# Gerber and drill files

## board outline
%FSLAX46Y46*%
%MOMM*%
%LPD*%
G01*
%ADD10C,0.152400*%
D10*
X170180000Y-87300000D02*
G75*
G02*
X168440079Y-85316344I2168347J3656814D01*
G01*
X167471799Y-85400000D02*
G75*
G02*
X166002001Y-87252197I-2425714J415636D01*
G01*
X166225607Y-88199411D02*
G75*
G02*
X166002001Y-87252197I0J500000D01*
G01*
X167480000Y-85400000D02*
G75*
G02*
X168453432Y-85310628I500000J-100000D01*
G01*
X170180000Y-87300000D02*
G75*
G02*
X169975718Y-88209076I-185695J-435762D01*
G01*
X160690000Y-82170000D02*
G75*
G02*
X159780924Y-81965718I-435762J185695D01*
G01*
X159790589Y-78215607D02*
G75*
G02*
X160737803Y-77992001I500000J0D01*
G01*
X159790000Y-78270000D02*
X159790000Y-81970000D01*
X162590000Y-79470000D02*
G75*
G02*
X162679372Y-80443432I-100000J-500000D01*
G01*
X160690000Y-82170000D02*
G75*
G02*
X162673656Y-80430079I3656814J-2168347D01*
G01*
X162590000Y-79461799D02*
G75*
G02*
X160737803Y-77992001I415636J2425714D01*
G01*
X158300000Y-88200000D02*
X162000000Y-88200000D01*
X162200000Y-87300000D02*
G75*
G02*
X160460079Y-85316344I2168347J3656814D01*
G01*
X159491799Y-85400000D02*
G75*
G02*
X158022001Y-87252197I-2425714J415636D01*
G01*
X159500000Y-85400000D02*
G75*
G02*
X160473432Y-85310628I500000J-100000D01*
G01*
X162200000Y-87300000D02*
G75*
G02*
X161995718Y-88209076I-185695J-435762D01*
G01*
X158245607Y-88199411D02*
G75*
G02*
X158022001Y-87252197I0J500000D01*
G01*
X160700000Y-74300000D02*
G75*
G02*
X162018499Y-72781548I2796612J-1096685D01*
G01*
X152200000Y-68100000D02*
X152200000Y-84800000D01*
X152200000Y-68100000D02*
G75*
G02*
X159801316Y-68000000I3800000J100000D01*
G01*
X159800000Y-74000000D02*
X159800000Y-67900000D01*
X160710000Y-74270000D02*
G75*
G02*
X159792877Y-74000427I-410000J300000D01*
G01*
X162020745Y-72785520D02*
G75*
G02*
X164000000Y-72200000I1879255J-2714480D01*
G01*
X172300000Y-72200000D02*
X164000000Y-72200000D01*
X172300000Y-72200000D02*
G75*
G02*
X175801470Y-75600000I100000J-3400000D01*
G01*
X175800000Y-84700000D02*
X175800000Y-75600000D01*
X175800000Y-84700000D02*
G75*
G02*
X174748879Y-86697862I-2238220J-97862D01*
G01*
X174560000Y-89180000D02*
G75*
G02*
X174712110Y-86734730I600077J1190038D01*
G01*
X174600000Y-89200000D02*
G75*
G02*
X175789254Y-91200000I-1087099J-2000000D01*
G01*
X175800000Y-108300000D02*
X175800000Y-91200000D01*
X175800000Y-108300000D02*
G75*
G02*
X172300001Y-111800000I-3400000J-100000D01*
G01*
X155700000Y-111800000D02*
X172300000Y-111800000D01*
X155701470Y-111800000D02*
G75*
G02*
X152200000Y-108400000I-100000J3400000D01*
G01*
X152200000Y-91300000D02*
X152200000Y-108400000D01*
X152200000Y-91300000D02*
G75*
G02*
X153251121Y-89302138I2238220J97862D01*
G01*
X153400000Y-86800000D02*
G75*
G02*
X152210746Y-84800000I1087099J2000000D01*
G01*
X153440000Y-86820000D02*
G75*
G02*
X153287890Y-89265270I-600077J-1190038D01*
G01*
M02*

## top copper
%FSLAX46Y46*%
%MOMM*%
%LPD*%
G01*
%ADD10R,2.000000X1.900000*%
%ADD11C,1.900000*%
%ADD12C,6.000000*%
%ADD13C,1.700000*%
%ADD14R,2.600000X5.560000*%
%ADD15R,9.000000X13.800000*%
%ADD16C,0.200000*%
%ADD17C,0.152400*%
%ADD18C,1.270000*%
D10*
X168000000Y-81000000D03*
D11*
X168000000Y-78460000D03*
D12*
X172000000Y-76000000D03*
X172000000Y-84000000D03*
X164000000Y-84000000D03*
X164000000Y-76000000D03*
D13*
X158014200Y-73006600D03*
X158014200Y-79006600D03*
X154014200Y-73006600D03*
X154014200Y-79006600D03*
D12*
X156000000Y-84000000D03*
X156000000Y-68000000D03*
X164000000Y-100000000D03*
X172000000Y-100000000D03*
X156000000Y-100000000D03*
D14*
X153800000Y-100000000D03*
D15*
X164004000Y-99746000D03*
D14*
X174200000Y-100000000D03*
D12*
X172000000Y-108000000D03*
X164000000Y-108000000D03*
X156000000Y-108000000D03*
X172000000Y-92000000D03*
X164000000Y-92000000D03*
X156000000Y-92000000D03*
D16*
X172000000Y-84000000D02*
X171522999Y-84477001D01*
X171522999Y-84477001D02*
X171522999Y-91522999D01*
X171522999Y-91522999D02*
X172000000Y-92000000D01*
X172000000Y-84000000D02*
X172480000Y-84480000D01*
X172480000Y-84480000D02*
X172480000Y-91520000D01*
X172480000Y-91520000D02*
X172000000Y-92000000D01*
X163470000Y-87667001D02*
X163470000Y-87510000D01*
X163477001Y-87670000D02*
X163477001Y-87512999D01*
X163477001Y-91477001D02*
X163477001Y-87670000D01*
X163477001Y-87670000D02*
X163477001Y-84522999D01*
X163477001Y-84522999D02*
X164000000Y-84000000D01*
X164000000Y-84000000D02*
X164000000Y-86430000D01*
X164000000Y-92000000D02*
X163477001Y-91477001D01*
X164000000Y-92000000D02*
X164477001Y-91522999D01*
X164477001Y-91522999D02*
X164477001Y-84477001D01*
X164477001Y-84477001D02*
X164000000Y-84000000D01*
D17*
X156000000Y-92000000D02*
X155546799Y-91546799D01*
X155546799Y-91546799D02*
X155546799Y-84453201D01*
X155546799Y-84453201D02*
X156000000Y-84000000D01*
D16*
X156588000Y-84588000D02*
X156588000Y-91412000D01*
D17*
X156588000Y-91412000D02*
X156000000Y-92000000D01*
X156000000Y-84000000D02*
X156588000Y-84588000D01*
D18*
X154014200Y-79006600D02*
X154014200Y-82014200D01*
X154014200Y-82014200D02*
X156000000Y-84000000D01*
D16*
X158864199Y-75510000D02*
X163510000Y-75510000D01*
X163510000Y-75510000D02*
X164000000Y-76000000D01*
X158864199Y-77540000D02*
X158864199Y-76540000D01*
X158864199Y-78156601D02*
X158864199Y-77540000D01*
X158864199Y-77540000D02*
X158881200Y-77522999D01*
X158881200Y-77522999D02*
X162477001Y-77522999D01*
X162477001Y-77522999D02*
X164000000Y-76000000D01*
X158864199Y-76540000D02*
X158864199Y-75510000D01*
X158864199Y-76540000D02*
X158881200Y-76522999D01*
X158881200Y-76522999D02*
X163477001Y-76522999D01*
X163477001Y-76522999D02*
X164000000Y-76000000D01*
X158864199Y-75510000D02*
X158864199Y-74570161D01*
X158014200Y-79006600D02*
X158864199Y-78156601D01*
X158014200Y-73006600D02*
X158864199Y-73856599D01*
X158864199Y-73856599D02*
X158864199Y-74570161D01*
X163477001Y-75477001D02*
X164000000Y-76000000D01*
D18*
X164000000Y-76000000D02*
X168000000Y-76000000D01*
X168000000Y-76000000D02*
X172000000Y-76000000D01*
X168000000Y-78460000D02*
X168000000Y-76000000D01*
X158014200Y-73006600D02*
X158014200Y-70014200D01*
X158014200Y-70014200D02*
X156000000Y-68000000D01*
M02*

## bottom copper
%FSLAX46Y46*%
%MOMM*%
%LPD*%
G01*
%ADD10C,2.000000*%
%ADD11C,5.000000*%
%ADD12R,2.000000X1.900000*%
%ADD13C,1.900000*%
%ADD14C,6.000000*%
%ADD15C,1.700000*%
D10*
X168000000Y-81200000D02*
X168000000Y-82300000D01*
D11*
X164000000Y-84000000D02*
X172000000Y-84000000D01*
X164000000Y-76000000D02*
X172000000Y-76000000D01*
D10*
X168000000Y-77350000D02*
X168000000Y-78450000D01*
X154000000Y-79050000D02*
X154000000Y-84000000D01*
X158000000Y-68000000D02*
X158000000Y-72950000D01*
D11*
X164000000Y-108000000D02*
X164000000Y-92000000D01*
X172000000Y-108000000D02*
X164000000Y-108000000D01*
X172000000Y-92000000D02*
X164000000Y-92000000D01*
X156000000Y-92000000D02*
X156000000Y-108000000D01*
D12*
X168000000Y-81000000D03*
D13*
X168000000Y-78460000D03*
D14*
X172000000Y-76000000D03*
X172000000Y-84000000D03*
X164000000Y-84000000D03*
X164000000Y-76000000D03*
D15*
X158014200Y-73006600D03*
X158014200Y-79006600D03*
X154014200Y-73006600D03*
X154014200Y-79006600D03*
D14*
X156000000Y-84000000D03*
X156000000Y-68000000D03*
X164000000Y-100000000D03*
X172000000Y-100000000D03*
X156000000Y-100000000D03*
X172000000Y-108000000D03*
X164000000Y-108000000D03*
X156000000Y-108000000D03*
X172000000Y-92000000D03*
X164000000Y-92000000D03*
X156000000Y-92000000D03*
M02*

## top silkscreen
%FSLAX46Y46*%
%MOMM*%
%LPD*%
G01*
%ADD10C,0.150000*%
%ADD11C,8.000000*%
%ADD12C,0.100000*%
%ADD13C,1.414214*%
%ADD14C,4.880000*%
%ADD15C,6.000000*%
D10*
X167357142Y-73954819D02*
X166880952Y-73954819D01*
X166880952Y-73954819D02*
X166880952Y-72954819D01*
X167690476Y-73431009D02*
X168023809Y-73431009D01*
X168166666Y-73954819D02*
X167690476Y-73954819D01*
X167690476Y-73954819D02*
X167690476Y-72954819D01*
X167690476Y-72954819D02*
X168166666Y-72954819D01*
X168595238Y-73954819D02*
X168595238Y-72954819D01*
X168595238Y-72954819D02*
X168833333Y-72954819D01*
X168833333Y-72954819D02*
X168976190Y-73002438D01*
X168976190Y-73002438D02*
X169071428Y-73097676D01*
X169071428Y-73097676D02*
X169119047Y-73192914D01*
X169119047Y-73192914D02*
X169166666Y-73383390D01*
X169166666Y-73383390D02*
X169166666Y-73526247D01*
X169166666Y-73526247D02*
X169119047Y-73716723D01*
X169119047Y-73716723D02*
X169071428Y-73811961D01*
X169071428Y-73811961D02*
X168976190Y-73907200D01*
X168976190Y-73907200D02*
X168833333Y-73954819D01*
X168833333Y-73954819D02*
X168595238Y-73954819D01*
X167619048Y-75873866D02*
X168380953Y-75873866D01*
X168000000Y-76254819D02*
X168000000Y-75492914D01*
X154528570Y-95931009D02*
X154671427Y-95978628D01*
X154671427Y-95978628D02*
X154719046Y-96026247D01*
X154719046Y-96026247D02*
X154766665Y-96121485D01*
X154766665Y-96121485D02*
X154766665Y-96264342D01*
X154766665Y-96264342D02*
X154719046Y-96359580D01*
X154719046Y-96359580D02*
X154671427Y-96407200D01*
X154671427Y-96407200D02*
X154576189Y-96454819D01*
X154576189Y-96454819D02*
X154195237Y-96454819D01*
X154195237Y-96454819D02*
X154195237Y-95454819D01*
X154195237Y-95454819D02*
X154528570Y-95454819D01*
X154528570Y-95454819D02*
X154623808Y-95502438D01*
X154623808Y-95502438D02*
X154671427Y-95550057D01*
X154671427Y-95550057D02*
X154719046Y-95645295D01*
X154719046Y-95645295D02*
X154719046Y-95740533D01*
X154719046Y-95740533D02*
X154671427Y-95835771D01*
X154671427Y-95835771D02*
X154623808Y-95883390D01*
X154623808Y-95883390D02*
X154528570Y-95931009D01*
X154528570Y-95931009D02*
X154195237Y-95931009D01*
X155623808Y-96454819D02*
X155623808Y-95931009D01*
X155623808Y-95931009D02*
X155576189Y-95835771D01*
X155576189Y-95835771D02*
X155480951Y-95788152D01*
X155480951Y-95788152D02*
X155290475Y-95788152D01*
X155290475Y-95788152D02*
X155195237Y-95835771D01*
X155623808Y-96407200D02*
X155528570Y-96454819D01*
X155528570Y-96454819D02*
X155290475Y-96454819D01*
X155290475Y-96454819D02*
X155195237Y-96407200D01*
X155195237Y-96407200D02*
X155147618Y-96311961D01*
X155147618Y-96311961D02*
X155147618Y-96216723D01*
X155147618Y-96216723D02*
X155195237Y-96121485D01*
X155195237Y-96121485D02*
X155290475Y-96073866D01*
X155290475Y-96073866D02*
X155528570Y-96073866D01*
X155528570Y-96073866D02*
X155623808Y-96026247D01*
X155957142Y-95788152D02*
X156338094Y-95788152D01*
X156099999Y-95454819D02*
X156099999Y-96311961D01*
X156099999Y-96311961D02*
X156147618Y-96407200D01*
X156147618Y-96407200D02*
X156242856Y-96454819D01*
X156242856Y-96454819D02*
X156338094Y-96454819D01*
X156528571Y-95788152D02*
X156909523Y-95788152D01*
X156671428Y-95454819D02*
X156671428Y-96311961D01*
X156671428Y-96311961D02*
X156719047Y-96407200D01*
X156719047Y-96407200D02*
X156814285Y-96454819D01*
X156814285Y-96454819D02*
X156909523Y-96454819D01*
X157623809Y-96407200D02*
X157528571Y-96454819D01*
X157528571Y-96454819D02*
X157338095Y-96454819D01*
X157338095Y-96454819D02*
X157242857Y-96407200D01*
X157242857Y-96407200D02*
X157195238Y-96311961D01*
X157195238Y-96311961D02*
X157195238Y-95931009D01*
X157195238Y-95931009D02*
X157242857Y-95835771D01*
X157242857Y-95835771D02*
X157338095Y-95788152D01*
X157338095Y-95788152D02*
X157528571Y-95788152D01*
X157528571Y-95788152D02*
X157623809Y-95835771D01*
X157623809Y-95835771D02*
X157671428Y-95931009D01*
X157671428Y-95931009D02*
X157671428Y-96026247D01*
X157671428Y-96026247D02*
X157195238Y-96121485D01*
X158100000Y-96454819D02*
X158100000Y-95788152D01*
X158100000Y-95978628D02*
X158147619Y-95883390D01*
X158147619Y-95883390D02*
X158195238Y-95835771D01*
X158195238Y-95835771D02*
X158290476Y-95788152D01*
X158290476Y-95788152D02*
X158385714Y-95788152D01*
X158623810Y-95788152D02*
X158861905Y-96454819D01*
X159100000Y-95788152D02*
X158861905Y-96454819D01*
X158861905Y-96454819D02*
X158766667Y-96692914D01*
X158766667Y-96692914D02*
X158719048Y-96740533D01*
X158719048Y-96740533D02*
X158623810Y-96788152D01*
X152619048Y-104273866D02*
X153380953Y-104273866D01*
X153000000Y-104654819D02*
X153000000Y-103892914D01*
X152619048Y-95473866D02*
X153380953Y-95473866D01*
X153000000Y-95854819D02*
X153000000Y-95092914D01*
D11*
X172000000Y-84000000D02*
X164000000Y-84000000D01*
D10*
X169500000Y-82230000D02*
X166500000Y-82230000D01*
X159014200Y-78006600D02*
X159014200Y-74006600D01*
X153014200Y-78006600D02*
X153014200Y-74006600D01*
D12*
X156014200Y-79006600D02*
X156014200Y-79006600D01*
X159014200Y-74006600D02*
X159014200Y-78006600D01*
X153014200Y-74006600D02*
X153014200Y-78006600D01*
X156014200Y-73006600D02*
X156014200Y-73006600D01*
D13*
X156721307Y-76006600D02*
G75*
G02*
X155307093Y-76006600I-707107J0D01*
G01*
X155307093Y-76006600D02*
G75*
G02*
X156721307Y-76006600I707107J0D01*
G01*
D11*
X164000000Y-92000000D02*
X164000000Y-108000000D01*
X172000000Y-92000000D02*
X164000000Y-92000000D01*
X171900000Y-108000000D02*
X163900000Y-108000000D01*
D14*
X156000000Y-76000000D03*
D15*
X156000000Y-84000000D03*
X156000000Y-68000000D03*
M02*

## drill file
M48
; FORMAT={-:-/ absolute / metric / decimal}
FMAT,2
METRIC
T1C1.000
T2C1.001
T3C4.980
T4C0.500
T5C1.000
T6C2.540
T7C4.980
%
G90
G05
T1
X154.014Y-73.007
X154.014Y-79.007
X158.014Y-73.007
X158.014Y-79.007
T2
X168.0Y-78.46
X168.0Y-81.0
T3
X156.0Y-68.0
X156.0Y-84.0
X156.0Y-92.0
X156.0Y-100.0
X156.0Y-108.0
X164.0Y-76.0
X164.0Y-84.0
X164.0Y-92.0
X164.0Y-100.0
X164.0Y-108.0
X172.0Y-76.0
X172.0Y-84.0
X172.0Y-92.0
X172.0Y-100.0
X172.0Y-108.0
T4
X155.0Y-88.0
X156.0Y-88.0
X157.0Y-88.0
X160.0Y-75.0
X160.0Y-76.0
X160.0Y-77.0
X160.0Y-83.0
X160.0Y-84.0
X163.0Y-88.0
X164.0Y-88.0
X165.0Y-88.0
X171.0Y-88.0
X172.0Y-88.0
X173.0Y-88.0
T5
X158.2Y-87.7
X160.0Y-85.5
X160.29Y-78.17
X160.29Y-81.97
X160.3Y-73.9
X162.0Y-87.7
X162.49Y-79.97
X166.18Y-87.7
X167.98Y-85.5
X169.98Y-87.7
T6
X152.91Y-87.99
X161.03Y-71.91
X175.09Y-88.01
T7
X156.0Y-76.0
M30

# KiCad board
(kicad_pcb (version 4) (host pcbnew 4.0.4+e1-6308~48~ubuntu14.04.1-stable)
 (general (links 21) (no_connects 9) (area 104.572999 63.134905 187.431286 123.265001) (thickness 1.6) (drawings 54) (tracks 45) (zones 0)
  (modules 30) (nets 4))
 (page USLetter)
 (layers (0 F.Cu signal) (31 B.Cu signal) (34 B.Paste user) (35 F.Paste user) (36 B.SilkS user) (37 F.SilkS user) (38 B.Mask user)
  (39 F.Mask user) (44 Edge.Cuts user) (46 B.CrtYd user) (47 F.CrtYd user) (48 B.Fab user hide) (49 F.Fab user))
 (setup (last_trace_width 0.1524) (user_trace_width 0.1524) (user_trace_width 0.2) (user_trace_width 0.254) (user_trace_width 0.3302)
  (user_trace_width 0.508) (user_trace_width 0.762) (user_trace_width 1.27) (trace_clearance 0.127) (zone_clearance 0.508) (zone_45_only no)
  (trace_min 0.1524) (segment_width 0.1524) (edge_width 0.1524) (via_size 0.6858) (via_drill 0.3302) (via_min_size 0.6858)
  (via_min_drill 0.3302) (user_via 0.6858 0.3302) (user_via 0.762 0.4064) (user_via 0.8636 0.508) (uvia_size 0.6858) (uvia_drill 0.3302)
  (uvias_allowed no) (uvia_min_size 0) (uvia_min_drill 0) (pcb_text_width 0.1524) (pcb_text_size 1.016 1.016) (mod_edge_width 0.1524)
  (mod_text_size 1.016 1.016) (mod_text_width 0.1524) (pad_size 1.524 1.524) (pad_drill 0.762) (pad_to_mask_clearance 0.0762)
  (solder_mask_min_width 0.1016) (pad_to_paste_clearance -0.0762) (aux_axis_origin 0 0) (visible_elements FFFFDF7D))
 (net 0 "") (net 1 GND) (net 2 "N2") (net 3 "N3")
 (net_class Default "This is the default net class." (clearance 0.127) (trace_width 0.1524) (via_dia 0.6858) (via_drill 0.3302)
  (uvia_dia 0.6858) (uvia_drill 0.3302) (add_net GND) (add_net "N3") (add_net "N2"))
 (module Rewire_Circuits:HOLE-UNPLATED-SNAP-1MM (layer F.Cu) (at 167.98 85.5 270)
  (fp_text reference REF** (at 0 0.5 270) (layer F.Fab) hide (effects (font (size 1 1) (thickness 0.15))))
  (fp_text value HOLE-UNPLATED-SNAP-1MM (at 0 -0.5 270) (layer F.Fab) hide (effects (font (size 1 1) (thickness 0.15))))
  (pad "" np_thru_hole circle (at 0 0 270) (size 1 1) (drill 1) (layers *.Cu)))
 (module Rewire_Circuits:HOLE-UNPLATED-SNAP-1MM (layer F.Cu) (at 166.18 87.7)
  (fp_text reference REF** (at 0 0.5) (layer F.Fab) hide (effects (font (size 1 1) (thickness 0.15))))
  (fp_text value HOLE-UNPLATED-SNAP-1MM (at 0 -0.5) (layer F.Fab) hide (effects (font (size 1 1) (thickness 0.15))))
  (pad "" np_thru_hole circle (at 0 0) (size 1 1) (drill 1) (layers *.Cu)))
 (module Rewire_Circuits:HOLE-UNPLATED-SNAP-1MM (layer F.Cu) (at 169.98 87.7)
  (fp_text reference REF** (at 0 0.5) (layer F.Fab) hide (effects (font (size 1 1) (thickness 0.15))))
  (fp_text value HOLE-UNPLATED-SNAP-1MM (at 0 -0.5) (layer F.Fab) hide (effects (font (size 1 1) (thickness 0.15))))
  (pad "" np_thru_hole circle (at 0 0) (size 1 1) (drill 1) (layers *.Cu)))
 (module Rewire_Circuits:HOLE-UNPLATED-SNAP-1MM (layer F.Cu) (at 162.49 79.97 180)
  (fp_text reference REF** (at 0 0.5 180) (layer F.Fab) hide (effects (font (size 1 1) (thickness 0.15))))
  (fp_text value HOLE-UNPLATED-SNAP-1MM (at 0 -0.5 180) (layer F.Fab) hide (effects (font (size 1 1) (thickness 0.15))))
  (pad "" np_thru_hole circle (at 0 0 180) (size 1 1) (drill 1) (layers *.Cu)))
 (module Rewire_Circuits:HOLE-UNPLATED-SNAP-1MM (layer F.Cu) (at 160.29 78.17 270)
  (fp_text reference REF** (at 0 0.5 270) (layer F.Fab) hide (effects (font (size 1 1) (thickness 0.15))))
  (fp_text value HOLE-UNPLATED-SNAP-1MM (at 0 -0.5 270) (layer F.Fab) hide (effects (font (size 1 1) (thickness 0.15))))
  (pad "" np_thru_hole circle (at 0 0 270) (size 1 1) (drill 1) (layers *.Cu)))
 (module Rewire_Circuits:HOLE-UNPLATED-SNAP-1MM (layer F.Cu) (at 160.29 81.97 270)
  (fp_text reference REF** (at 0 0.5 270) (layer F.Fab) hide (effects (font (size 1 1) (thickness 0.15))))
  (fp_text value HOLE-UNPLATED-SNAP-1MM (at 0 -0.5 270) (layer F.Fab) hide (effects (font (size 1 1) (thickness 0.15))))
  (pad "" np_thru_hole circle (at 0 0 270) (size 1 1) (drill 1) (layers *.Cu)))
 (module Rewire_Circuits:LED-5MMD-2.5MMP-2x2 (layer F.Cu) (at 168 80 180)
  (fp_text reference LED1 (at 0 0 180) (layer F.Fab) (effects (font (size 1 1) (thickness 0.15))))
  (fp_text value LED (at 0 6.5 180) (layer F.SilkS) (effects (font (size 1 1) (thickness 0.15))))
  (fp_line (start 0 -1.2) (end 0 -2.3) (layer B.Cu) (width 2))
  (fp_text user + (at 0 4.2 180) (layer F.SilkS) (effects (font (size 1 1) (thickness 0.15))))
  (fp_line (start -4 -4) (end 4 -4) (layer F.SilkS) (width 8))
  (fp_line (start -1.5 -2.23) (end 1.5 -2.23) (layer F.SilkS) (width 0.15)) (fp_line (start 4 -4) (end -4 -4) (layer B.Cu) (width 5))
  (fp_line (start 4 4) (end -4 4) (layer B.Cu) (width 5)) (fp_line (start 0 2.65) (end 0 1.55) (layer B.Cu) (width 2))
  (pad - thru_hole rect (at 0 -1 180) (size 2 1.9) (drill 1.00076) (layers *.Cu *.Mask) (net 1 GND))
  (pad + thru_hole circle (at 0 1.54 90) (size 1.9 1.9) (drill 1.00076) (layers *.Cu *.Mask) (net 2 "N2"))
  (pad + thru_hole circle (at -4 4 180) (size 6 6) (drill 4.98) (layers *.Cu *.Mask) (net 2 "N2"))
  (pad - thru_hole circle (at -4 -4 180) (size 6 6) (drill 4.98) (layers *.Cu *.Mask) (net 1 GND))
  (pad - thru_hole circle (at 4 -4 180) (size 6 6) (drill 4.98) (layers *.Cu *.Mask) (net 1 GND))
  (pad + thru_hole circle (at 4 4 180) (size 6 6) (drill 4.98) (layers *.Cu *.Mask) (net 2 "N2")))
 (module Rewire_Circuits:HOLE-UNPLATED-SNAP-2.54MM (layer F.Cu) (at 161.03 71.91)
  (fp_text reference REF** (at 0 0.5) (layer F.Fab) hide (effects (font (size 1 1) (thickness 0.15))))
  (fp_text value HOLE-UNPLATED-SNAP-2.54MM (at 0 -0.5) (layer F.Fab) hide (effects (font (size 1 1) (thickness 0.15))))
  (pad "" np_thru_hole circle (at 0 0) (size 2.54 2.54) (drill 2.54) (layers *.Cu)))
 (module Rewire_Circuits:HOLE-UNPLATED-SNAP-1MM (layer F.Cu) (at 160 85.5 270)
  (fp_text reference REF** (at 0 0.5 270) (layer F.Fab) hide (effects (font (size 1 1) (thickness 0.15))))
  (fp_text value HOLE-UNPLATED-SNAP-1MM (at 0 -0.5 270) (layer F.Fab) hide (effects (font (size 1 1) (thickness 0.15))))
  (pad "" np_thru_hole circle (at 0 0 270) (size 1 1) (drill 1) (layers *.Cu)))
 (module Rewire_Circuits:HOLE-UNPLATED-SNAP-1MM (layer F.Cu) (at 160.3 73.9)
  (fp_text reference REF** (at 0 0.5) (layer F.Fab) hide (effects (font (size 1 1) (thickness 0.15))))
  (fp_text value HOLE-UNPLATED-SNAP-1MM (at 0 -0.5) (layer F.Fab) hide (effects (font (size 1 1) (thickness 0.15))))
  (pad "" np_thru_hole circle (at 0 0) (size 1 1) (drill 1) (layers *.Cu)))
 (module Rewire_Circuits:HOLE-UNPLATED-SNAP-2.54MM (layer F.Cu) (at 175.09 88.01 180)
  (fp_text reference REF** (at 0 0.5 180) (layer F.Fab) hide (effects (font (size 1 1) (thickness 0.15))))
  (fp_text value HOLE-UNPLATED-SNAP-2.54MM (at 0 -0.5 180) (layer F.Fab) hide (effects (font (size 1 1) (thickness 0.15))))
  (pad "" np_thru_hole circle (at 0 0 180) (size 2.54 2.54) (drill 2.54) (layers *.Cu)))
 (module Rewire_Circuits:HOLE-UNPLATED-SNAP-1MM (layer F.Cu) (at 162 87.7)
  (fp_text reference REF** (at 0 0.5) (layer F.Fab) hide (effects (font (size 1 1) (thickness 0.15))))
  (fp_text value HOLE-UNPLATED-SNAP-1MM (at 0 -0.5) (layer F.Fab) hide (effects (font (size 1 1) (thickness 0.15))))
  (pad "" np_thru_hole circle (at 0 0) (size 1 1) (drill 1) (layers *.Cu)))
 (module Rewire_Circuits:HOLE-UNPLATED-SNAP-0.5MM (layer F.Cu) (at 163 88 180)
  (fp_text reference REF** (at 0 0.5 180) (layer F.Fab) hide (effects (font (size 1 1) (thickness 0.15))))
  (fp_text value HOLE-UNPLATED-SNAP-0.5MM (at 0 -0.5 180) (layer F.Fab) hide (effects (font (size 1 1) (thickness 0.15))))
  (pad "" np_thru_hole circle (at 0 0 180) (size 0.5 0.5) (drill 0.5) (layers *.Cu)))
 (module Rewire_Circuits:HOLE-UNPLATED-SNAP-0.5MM (layer F.Cu) (at 164 88 180)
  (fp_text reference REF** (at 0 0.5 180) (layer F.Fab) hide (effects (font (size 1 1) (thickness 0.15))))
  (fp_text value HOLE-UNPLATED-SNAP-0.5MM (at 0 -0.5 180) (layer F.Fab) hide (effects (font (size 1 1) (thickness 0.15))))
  (pad "" np_thru_hole circle (at 0 0 180) (size 0.5 0.5) (drill 0.5) (layers *.Cu)))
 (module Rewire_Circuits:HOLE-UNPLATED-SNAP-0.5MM (layer F.Cu) (at 173 88 180)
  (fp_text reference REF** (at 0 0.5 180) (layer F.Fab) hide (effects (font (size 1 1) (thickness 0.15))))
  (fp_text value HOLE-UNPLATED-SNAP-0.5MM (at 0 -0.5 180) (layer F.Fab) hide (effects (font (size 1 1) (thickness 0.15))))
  (pad "" np_thru_hole circle (at 0 0 180) (size 0.5 0.5) (drill 0.5) (layers *.Cu)))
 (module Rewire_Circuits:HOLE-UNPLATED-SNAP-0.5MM (layer F.Cu) (at 172 88 180)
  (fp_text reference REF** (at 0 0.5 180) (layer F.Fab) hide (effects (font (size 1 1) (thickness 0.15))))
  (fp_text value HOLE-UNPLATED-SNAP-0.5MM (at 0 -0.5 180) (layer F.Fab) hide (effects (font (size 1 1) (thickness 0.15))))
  (pad "" np_thru_hole circle (at 0 0 180) (size 0.5 0.5) (drill 0.5) (layers *.Cu)))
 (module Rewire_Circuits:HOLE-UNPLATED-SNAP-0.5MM (layer F.Cu) (at 171 88 180)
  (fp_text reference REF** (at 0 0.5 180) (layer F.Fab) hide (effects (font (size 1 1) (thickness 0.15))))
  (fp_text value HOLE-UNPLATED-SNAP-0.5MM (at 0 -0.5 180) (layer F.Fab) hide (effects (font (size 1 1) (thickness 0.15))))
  (pad "" np_thru_hole circle (at 0 0 180) (size 0.5 0.5) (drill 0.5) (layers *.Cu)))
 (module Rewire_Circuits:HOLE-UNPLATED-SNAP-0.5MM (layer F.Cu) (at 165 88 180)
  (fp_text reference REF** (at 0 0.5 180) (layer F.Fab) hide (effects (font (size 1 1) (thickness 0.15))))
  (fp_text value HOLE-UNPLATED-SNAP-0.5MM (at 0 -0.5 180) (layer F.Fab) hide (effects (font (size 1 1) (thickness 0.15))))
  (pad "" np_thru_hole circle (at 0 0 180) (size 0.5 0.5) (drill 0.5) (layers *.Cu)))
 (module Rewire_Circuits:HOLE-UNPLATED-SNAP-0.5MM (layer F.Cu) (at 160 75 90)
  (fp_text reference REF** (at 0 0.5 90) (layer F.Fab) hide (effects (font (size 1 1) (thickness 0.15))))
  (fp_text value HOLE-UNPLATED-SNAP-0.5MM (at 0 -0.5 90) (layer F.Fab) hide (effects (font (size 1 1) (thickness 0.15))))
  (pad "" np_thru_hole circle (at 0 0 90) (size 0.5 0.5) (drill 0.5) (layers *.Cu)))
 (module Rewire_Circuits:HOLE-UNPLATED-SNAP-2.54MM (layer F.Cu) (at 152.91 87.99)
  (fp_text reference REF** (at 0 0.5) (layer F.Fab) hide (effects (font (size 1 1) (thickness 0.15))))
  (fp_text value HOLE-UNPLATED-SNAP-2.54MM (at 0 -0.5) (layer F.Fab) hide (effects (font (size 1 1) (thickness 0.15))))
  (pad "" np_thru_hole circle (at 0 0) (size 2.54 2.54) (drill 2.54) (layers *.Cu)))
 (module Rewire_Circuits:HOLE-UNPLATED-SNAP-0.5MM (layer F.Cu) (at 160 84 90)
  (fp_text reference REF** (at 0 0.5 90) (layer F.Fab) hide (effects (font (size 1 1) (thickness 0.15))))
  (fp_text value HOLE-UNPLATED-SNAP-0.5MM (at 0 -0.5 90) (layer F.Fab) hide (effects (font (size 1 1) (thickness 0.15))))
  (pad "" np_thru_hole circle (at 0 0 90) (size 0.5 0.5) (drill 0.5) (layers *.Cu)))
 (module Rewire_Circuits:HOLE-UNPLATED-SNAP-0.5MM (layer F.Cu) (at 160 83 90)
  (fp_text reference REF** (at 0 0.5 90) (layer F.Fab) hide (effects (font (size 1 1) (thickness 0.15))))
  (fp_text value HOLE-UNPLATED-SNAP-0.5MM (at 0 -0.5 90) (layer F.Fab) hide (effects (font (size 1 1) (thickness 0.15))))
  (pad "" np_thru_hole circle (at 0 0 90) (size 0.5 0.5) (drill 0.5) (layers *.Cu)))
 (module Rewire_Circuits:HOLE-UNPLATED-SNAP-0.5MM (layer F.Cu) (at 160 76 90)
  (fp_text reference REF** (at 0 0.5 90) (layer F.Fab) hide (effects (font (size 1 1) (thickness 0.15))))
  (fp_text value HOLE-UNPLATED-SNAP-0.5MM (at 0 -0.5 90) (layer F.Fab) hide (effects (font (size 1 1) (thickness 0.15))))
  (pad "" np_thru_hole circle (at 0 0 90) (size 0.5 0.5) (drill 0.5) (layers *.Cu)))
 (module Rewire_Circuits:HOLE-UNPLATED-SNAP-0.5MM (layer F.Cu) (at 160 77 90)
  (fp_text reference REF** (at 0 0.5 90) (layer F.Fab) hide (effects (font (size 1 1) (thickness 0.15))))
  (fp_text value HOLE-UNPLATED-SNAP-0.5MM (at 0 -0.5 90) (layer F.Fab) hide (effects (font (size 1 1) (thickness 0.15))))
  (pad "" np_thru_hole circle (at 0 0 90) (size 0.5 0.5) (drill 0.5) (layers *.Cu)))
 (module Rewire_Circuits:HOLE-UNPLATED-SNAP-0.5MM (layer F.Cu) (at 155 88)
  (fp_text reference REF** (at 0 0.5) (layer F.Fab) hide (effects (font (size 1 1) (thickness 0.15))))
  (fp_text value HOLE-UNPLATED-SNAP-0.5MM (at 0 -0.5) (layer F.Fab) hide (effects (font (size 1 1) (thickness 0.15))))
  (pad "" np_thru_hole circle (at 0 0) (size 0.5 0.5) (drill 0.5) (layers *.Cu)))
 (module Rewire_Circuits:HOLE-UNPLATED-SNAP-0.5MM (layer F.Cu) (at 157 88)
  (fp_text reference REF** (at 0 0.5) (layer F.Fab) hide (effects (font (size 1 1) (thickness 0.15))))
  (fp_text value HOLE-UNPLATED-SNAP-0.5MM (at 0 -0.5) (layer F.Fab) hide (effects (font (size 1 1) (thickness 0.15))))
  (pad "" np_thru_hole circle (at 0 0) (size 0.5 0.5) (drill 0.5) (layers *.Cu)))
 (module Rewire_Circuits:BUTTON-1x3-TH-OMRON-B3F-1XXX (layer F.Cu) (at 156 76 90)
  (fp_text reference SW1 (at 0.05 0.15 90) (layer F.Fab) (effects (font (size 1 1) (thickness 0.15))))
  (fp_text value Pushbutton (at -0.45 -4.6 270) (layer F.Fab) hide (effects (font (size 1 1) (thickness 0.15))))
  (fp_line (start -3.05 -2) (end -8 -2) (layer B.Cu) (width 2))
  (fp_line (start -2.0066 3.0142) (end 1.9934 3.0142) (layer F.SilkS) (width 0.15))
  (fp_line (start -2.0066 -2.9858) (end 1.9934 -2.9858) (layer F.SilkS) (width 0.15))
  (fp_line (start -3.0066 0.0142) (end -3.0066 0.0142) (layer F.SilkS) (width 0))
  (fp_line (start 1.9934 3.0142) (end -2.0066 3.0142) (layer F.SilkS) (width 0))
  (fp_line (start 1.9934 -2.9858) (end -2.0066 -2.9858) (layer F.SilkS) (width 0))
  (fp_line (start 2.9934 0.0142) (end 2.9934 0.0142) (layer F.SilkS) (width 0))
  (fp_circle (center -0.0066 0.0142) (end 0.9934 1.0142) (layer F.SilkS) (width 0))
  (fp_line (start 8 2) (end 3.05 2) (layer B.Cu) (width 2))
  (pad 2 thru_hole circle (at 2.9934 2.0142 90) (size 1.7 1.7) (drill 1) (layers *.Cu *.Mask) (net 2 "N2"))
  (pad 2 thru_hole circle (at -3.0066 2.0142 90) (size 1.7 1.7) (drill 1) (layers *.Cu *.Mask) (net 2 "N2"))
  (pad 1 thru_hole circle (at 2.9934 -1.9858 90) (size 1.7 1.7) (drill 1) (layers *.Cu *.Mask) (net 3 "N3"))
  (pad 1 thru_hole circle (at -3.0066 -1.9858 90) (size 1.7 1.7) (drill 1) (layers *.Cu *.Mask) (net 3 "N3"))
  (pad "" np_thru_hole circle (at 0 0 90) (size 4.88 4.88) (drill 4.98) (layers *.Cu *.Mask F.SilkS))
  (pad 1 thru_hole circle (at -8 0 90) (size 6 6) (drill 4.98) (layers *.Cu *.Mask F.SilkS) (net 3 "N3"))
  (pad 2 thru_hole circle (at 8 0 90) (size 6 6) (drill 4.98) (layers *.Cu *.Mask F.SilkS) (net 2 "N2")))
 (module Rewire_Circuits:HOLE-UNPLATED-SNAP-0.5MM (layer F.Cu) (at 156 88)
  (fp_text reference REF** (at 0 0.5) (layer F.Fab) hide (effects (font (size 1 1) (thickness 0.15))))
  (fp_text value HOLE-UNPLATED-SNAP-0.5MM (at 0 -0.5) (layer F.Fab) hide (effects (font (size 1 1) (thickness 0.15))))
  (pad "" np_thru_hole circle (at 0 0) (size 0.5 0.5) (drill 0.5) (layers *.Cu)))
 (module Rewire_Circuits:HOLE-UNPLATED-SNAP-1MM (layer F.Cu) (at 158.2 87.7)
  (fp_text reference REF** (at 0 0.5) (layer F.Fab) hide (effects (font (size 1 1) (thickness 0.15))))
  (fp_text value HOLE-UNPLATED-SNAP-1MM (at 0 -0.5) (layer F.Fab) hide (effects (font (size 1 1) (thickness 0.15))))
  (pad "" np_thru_hole circle (at 0 0) (size 1 1) (drill 1) (layers *.Cu)))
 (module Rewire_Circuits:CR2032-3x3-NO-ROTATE (layer F.Cu) (at 164 100 180)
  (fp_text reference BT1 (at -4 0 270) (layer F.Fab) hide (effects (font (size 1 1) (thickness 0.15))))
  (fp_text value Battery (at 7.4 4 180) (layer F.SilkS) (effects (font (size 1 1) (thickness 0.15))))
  (fp_line (start 0 8) (end 0 -8) (layer F.SilkS) (width 8)) (fp_line (start 0 -8) (end 0 8) (layer B.Cu) (width 5))
  (fp_line (start -8 -8) (end 0 -8) (layer B.Cu) (width 5)) (fp_line (start -8 8) (end 0 8) (layer B.Cu) (width 5))
  (fp_line (start 8 8) (end 8 -8) (layer B.Cu) (width 5))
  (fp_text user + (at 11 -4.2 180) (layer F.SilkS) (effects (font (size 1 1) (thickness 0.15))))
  (fp_line (start -8 8) (end 0 8) (layer F.SilkS) (width 8))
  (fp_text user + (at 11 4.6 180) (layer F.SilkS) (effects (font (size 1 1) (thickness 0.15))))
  (fp_line (start -7.9 -8) (end 0.1 -8) (layer F.SilkS) (width 8))
  (pad GND thru_hole circle (at 0 0 180) (size 6 6) (drill 4.98) (layers *.Cu *.Mask) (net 1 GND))
  (pad + thru_hole circle (at -8 0 180) (size 6 6) (drill 4.98) (layers *.Cu *.Mask) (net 3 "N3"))
  (pad + thru_hole circle (at 8 0 180) (size 6 6) (drill 4.98) (layers *.Cu *.Mask) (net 3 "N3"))
  (pad + smd rect (at 10.2 0 180) (size 2.6 5.56) (layers F.Cu F.Paste F.Mask) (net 3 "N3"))
  (pad GND smd rect (at -0.004 0.254 180) (size 9 13.8) (layers F.Cu F.Paste F.Mask) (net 1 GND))
  (pad + smd rect (at -10.2 0 180) (size 2.6 5.56) (layers F.Cu F.Paste F.Mask) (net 3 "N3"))
  (pad GND thru_hole circle (at -8 -8 180) (size 6 6) (drill 4.98) (layers *.Cu *.Mask) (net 1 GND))
  (pad GND thru_hole circle (at 0 -8 180) (size 6 6) (drill 4.98) (layers *.Cu *.Mask) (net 1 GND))
  (pad + thru_hole circle (at 8 -8 180) (size 6 6) (drill 4.98) (layers *.Cu *.Mask) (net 3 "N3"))
  (pad GND thru_hole circle (at -8 8 180) (size 6 6) (drill 4.98) (layers *.Cu *.Mask) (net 1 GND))
  (pad GND thru_hole circle (at 0 8 180) (size 6 6) (drill 4.98) (layers *.Cu *.Mask) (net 1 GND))
  (pad + thru_hole circle (at 8 8 180) (size 6 6) (drill 4.98) (layers *.Cu *.Mask) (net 3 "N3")))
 (gr_arc (start 172.348347 83.643186) (end 170.18 87.3) (angle 36.15760514) (layer Edge.Cuts) (width 0.1524))
 (gr_arc (start 165.046085 84.984364) (end 167.471799 85.4) (angle 57.42107103) (layer Edge.Cuts) (width 0.1524))
 (gr_arc (start 166.225607 87.699411) (end 166.225607 88.199411) (angle 153.4350001) (layer Edge.Cuts) (width 0.1524))
 (gr_arc (start 167.98 85.5) (end 167.48 85.4) (angle 146.8886998) (layer Edge.Cuts) (width 0.1524))
 (gr_arc (start 169.994305 87.735762) (end 170.18 87.3) (angle 159.1681201) (layer Edge.Cuts) (width 0.1524))
 (gr_arc (start 160.254238 81.984305) (end 160.69 82.17) (angle 159.1681201) (layer Edge.Cuts) (width 0.1524))
 (gr_arc (start 160.290589 78.215607) (end 159.790589 78.215607) (angle 153.4350001) (layer Edge.Cuts) (width 0.1524))
 (gr_line (start 159.79 78.27) (end 159.79 81.97) (layer Edge.Cuts) (width 0.1524))
 (gr_arc (start 162.49 79.97) (end 162.59 79.47) (angle 146.8886998) (layer Edge.Cuts) (width 0.1524))
 (gr_arc (start 164.346814 84.338347) (end 160.69 82.17) (angle 36.15760514) (layer Edge.Cuts) (width 0.1524))
 (gr_arc (start 163.005636 77.036085) (end 162.59 79.461799) (angle 57.42107103) (layer Edge.Cuts) (width 0.1524))
 (gr_line (start 158.3 88.2) (end 162 88.2) (layer Edge.Cuts) (width 0.1524))
 (gr_arc (start 164.368347 83.643186) (end 162.2 87.3) (angle 36.15760514) (layer Edge.Cuts) (width 0.1524))
 (gr_arc (start 157.066085 84.984364) (end 159.491799 85.4) (angle 57.42107103) (layer Edge.Cuts) (width 0.1524))
 (gr_arc (start 160 85.5) (end 159.5 85.4) (angle 146.8886998) (layer Edge.Cuts) (width 0.1524))
 (gr_arc (start 162.014305 87.735762) (end 162.2 87.3) (angle 159.1681201) (layer Edge.Cuts) (width 0.1524))
 (gr_arc (start 158.245607 87.699411) (end 158.245607 88.199411) (angle 153.4350001) (layer Edge.Cuts) (width 0.1524))
 (gr_arc (start 163.496612 75.396685) (end 160.7 74.3) (angle 39.11172728) (layer Edge.Cuts) (width 0.1524))
 (gr_line (start 152.2 68.1) (end 152.2 84.8) (layer Edge.Cuts) (width 0.1524))
 (gr_arc (start 156 68) (end 152.2 68.1) (angle 181.5074358) (layer Edge.Cuts) (width 0.1524))
 (gr_line (start 159.8 74) (end 159.8 67.9) (layer Edge.Cuts) (width 0.1524))
 (gr_arc (start 160.3 73.97) (end 160.71 74.27) (angle 140.3732051) (layer Edge.Cuts) (width 0.1524))
 (gr_arc (start 163.9 75.5) (end 164 72.2) (angle -36.43084824) (layer Edge.Cuts) (width 0.1524))
 (gr_line (start 172.3 72.2) (end 164 72.2) (layer Edge.Cuts) (width 0.1524))
 (gr_arc (start 172.4 75.6) (end 172.3 72.2) (angle 91.68468432) (layer Edge.Cuts) (width 0.1524))
 (gr_line (start 175.8 84.7) (end 175.8 75.6) (layer Edge.Cuts) (width 0.1524))
 (gr_arc (start 173.56178 84.797862) (end 174.748879 86.697862) (angle -60.50687109) (layer Edge.Cuts) (width 0.1524))
 (gr_arc (start 175.160077 87.989962) (end 174.56 89.18) (angle 133.6) (layer Edge.Cuts) (width 0.1524))
 (gr_arc (start 173.512901 91.2) (end 174.6 89.2) (angle 61.47373049) (layer Edge.Cuts) (width 0.1524))
 (gr_line (start 175.8 108.3) (end 175.8 91.2) (layer Edge.Cuts) (width 0.1524))
 (gr_arc (start 172.4 108.4) (end 175.8 108.3) (angle 93.36935229) (layer Edge.Cuts) (width 0.1524))
 (gr_line (start 155.7 111.8) (end 172.3 111.8) (layer Edge.Cuts) (width 0.1524))
 (gr_arc (start 155.60147 108.4) (end 155.70147 111.8) (angle 91.68468432) (layer Edge.Cuts) (width 0.1524))
 (gr_line (start 152.2 91.3) (end 152.2 108.4) (layer Edge.Cuts) (width 0.1524))
 (gr_arc (start 154.43822 91.202138) (end 153.251121 89.302138) (angle -60.50687109) (layer Edge.Cuts) (width 0.1524))
 (gr_arc (start 154.487099 84.8) (end 153.4 86.8) (angle 61.47373049) (layer Edge.Cuts) (width 0.1524))
 (gr_arc (start 152.839923 88.010038) (end 153.44 86.82) (angle 133.6) (layer Edge.Cuts) (width 0.1524))
 (segment (start 172 84) (end 171.522999 84.477001) (width 0.2) (layer F.Cu) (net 1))
 (segment (start 171.522999 84.477001) (end 171.522999 91.522999) (width 0.2) (layer F.Cu) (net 1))
 (segment (start 171.522999 91.522999) (end 172 92) (width 0.2) (layer F.Cu) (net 1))
 (segment (start 172 84) (end 172.48 84.48) (width 0.2) (layer F.Cu) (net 1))
 (segment (start 172.48 84.48) (end 172.48 91.52) (width 0.2) (layer F.Cu) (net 1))
 (segment (start 172.48 91.52) (end 172 92) (width 0.2) (layer F.Cu) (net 1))
 (segment (start 163.47 87.667001) (end 163.47 87.51) (width 0.2) (layer F.Cu) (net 1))
 (segment (start 163.477001 87.67) (end 163.477001 87.512999) (width 0.2) (layer F.Cu) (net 1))
 (segment (start 163.477001 91.477001) (end 163.477001 87.67) (width 0.2) (layer F.Cu) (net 1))
 (segment (start 163.477001 87.67) (end 163.477001 84.522999) (width 0.2) (layer F.Cu) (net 1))
 (segment (start 163.477001 84.522999) (end 164 84) (width 0.2) (layer F.Cu) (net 1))
 (segment (start 164 84) (end 164 86.43) (width 0.2) (layer F.Cu) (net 1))
 (segment (start 164 92) (end 163.477001 91.477001) (width 0.2) (layer F.Cu) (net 1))
 (segment (start 164 92) (end 164.477001 91.522999) (width 0.2) (layer F.Cu) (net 1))
 (segment (start 164.477001 91.522999) (end 164.477001 84.477001) (width 0.2) (layer F.Cu) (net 1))
 (segment (start 164.477001 84.477001) (end 164 84) (width 0.2) (layer F.Cu) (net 1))
 (segment (start 156 92) (end 155.546799 91.546799) (width 0.1524) (layer F.Cu) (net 3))
 (segment (start 155.546799 91.546799) (end 155.546799 84.453201) (width 0.1524) (layer F.Cu) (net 3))
 (segment (start 155.546799 84.453201) (end 156 84) (width 0.1524) (layer F.Cu) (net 3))
 (segment (start 156.588 84.588) (end 156.588 91.412) (width 0.2) (layer F.Cu) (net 3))
 (segment (start 156.588 91.412) (end 156 92) (width 0.1524) (layer F.Cu) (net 3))
 (segment (start 156 84) (end 156.588 84.588) (width 0.1524) (layer F.Cu) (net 3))
 (segment (start 154.0142 79.0066) (end 154.0142 82.0142) (width 1.27) (layer F.Cu) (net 3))
 (segment (start 154.0142 82.0142) (end 156 84) (width 1.27) (layer F.Cu) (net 3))
 (segment (start 158.864199 75.51) (end 163.51 75.51) (width 0.2) (layer F.Cu) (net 2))
 (segment (start 163.51 75.51) (end 164 76) (width 0.2) (layer F.Cu) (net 2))
 (segment (start 158.864199 77.54) (end 158.864199 76.54) (width 0.2) (layer F.Cu) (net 2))
 (segment (start 158.864199 78.156601) (end 158.864199 77.54) (width 0.2) (layer F.Cu) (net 2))
 (segment (start 158.864199 77.54) (end 158.8812 77.522999) (width 0.2) (layer F.Cu) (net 2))
 (segment (start 158.8812 77.522999) (end 162.477001 77.522999) (width 0.2) (layer F.Cu) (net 2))
 (segment (start 162.477001 77.522999) (end 164 76) (width 0.2) (layer F.Cu) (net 2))
 (segment (start 158.864199 76.54) (end 158.864199 75.51) (width 0.2) (layer F.Cu) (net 2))
 (segment (start 158.864199 76.54) (end 158.8812 76.522999) (width 0.2) (layer F.Cu) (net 2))
 (segment (start 158.8812 76.522999) (end 163.477001 76.522999) (width 0.2) (layer F.Cu) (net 2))
 (segment (start 163.477001 76.522999) (end 164 76) (width 0.2) (layer F.Cu) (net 2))
 (segment (start 158.864199 75.51) (end 158.864199 74.570161) (width 0.2) (layer F.Cu) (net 2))
 (segment (start 158.0142 79.0066) (end 158.864199 78.156601) (width 0.2) (layer F.Cu) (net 2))
 (segment (start 158.0142 73.0066) (end 158.864199 73.856599) (width 0.2) (layer F.Cu) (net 2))
 (segment (start 158.864199 73.856599) (end 158.864199 74.570161) (width 0.2) (layer F.Cu) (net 2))
 (segment (start 163.477001 75.477001) (end 164 76) (width 0.2) (layer F.Cu) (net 2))
 (segment (start 164 76) (end 168 76) (width 1.27) (layer F.Cu) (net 2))
 (segment (start 168 76) (end 172 76) (width 1.27) (layer F.Cu) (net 2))
 (segment (start 168 78.46) (end 168 76) (width 1.27) (layer F.Cu) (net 2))
 (segment (start 158.0142 73.0066) (end 158.0142 70.0142) (width 1.27) (layer F.Cu) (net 2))
 (segment (start 158.0142 70.0142) (end 156 68) (width 1.27) (layer F.Cu) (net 2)))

